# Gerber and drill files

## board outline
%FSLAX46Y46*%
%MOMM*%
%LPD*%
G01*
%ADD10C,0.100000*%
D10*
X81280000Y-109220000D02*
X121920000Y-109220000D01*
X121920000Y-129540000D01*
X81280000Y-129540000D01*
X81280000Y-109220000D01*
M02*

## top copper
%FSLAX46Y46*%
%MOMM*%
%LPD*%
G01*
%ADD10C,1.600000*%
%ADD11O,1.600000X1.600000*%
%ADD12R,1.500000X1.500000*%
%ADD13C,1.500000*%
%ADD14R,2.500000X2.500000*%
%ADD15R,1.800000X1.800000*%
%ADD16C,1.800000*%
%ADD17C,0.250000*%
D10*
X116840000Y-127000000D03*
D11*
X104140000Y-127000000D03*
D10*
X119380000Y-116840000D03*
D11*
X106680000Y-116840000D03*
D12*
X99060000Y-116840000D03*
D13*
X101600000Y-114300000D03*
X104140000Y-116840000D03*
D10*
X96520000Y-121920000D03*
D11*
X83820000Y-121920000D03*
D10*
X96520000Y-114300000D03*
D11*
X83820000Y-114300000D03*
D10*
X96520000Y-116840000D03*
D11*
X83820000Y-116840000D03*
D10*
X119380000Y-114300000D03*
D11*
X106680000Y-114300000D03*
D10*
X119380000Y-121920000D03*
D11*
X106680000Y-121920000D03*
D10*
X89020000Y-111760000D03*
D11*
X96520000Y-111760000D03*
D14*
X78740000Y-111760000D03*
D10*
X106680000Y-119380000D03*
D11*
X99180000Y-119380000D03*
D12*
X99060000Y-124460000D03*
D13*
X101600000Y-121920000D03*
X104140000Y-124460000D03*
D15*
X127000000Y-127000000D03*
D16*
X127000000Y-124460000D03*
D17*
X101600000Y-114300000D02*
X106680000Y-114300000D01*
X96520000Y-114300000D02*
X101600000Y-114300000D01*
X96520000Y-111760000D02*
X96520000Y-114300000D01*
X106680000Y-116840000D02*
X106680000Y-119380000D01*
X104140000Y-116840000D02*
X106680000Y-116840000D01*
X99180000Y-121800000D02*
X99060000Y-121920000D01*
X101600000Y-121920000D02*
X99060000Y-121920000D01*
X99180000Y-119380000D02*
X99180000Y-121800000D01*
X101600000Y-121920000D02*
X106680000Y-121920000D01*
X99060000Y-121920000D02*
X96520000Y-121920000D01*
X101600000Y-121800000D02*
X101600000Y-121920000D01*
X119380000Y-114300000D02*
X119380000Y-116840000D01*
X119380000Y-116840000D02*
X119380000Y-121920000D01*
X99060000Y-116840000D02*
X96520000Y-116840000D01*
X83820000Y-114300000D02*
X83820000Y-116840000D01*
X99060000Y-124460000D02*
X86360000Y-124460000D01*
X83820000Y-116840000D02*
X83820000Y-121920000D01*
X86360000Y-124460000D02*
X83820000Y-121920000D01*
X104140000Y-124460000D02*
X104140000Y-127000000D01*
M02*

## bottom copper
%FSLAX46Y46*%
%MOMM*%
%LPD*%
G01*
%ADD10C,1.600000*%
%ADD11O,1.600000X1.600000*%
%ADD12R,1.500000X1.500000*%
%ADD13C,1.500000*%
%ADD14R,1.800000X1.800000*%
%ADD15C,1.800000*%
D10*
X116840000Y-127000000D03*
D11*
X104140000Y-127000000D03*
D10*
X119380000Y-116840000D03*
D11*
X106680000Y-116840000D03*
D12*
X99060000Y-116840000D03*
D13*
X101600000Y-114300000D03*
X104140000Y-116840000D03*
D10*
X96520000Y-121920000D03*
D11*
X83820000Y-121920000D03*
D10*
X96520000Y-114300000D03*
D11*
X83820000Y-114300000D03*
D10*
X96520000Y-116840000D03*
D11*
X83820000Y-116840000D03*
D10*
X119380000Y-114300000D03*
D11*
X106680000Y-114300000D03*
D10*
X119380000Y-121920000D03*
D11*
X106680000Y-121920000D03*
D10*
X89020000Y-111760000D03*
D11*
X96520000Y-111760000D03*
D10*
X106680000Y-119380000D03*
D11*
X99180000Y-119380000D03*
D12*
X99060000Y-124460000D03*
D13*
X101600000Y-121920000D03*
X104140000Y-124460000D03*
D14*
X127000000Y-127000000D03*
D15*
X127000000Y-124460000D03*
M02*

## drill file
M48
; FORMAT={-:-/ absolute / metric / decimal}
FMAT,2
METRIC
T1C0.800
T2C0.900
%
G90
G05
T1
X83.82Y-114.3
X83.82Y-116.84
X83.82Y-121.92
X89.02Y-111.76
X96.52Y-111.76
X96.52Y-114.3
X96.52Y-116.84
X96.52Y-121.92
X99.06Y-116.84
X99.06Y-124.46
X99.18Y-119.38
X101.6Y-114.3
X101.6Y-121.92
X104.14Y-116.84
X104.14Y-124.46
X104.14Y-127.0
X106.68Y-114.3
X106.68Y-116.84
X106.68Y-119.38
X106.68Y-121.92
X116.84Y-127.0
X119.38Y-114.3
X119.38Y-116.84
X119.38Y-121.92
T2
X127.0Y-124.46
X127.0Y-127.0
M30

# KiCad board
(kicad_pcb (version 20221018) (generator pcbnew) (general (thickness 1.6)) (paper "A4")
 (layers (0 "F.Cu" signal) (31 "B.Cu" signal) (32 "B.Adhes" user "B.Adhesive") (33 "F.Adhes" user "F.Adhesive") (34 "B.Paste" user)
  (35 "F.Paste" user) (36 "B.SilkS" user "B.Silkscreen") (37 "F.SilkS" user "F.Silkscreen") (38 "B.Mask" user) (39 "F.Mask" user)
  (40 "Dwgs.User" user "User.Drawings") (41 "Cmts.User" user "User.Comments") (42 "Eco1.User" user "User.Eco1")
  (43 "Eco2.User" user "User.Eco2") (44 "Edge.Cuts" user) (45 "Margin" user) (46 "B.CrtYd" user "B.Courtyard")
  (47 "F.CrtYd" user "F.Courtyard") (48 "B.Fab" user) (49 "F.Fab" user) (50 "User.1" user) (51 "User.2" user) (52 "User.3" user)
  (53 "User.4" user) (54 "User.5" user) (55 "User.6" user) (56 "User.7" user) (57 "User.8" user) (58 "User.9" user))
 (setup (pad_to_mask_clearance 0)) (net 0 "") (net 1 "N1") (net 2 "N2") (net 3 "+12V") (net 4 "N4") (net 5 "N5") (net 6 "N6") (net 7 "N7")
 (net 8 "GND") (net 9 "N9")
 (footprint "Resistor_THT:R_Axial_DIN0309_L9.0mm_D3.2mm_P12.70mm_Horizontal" (layer "F.Cu") (at 116.84 127 180)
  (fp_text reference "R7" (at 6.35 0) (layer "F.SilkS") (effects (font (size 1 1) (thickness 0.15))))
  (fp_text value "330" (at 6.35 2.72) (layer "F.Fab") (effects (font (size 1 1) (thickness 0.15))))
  (pad "1" thru_hole circle (at 0 0 180) (size 1.6 1.6) (drill 0.8) (layers "*.Cu" "*.Mask") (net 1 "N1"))
  (pad "2" thru_hole oval (at 12.7 0 180) (size 1.6 1.6) (drill 0.8) (layers "*.Cu" "*.Mask") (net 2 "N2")))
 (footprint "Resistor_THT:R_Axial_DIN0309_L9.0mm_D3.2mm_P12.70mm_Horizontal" (layer "F.Cu") (at 119.38 116.84 180)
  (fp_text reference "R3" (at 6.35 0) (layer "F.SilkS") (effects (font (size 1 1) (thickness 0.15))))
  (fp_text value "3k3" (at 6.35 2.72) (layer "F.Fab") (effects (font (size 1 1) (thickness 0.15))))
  (pad "1" thru_hole circle (at 0 0 180) (size 1.6 1.6) (drill 0.8) (layers "*.Cu" "*.Mask") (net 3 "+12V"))
  (pad "2" thru_hole oval (at 12.7 0 180) (size 1.6 1.6) (drill 0.8) (layers "*.Cu" "*.Mask") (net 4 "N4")))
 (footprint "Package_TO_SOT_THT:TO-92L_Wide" (layer "F.Cu") (at 99.06 116.84)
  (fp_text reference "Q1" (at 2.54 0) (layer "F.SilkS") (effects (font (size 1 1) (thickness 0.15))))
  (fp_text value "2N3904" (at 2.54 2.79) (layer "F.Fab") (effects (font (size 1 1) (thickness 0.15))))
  (pad "1" thru_hole rect (at 0 0) (size 1.5 1.5) (drill 0.8) (layers "*.Cu" "*.Mask") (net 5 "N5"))
  (pad "2" thru_hole circle (at 2.54 -2.54) (size 1.5 1.5) (drill 0.8) (layers "*.Cu" "*.Mask") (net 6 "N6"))
  (pad "3" thru_hole circle (at 5.08 0) (size 1.5 1.5) (drill 0.8) (layers "*.Cu" "*.Mask") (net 4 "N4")))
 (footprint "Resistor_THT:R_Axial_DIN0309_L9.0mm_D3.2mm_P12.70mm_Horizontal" (layer "F.Cu") (at 96.52 121.92 180)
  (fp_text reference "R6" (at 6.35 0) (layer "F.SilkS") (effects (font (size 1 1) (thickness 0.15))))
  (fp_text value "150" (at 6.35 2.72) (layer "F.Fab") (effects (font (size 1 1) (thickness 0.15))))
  (pad "1" thru_hole circle (at 0 0 180) (size 1.6 1.6) (drill 0.8) (layers "*.Cu" "*.Mask") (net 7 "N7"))
  (pad "2" thru_hole oval (at 12.7 0 180) (size 1.6 1.6) (drill 0.8) (layers "*.Cu" "*.Mask") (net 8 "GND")))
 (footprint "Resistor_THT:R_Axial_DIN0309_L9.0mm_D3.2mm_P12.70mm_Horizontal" (layer "F.Cu") (at 96.52 114.3 180)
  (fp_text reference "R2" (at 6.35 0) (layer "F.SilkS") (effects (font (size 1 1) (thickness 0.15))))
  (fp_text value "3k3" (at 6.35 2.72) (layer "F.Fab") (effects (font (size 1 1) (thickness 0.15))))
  (pad "1" thru_hole circle (at 0 0 180) (size 1.6 1.6) (drill 0.8) (layers "*.Cu" "*.Mask") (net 6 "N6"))
  (pad "2" thru_hole oval (at 12.7 0 180) (size 1.6 1.6) (drill 0.8) (layers "*.Cu" "*.Mask") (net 8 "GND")))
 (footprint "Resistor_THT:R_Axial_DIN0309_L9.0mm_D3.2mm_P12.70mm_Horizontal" (layer "F.Cu") (at 96.52 116.84 180)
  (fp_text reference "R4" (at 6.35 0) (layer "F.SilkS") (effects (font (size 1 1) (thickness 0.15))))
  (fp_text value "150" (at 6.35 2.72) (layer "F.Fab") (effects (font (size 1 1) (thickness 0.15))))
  (pad "1" thru_hole circle (at 0 0 180) (size 1.6 1.6) (drill 0.8) (layers "*.Cu" "*.Mask") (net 5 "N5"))
  (pad "2" thru_hole oval (at 12.7 0 180) (size 1.6 1.6) (drill 0.8) (layers "*.Cu" "*.Mask") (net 8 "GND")))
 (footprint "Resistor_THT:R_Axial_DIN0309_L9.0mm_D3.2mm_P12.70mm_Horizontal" (layer "F.Cu") (at 119.38 114.3 180)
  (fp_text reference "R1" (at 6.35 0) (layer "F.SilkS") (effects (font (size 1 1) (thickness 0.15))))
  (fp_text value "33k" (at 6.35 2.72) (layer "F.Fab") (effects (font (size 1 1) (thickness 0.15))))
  (pad "1" thru_hole circle (at 0 0 180) (size 1.6 1.6) (drill 0.8) (layers "*.Cu" "*.Mask") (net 3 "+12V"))
  (pad "2" thru_hole oval (at 12.7 0 180) (size 1.6 1.6) (drill 0.8) (layers "*.Cu" "*.Mask") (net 6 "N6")))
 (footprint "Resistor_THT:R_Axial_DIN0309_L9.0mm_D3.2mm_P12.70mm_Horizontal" (layer "F.Cu") (at 119.38 121.92 180)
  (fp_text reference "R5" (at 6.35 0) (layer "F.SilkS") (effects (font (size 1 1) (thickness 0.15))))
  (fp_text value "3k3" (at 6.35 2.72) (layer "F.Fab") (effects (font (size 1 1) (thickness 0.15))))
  (pad "1" thru_hole circle (at 0 0 180) (size 1.6 1.6) (drill 0.8) (layers "*.Cu" "*.Mask") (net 3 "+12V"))
  (pad "2" thru_hole oval (at 12.7 0 180) (size 1.6 1.6) (drill 0.8) (layers "*.Cu" "*.Mask") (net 7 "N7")))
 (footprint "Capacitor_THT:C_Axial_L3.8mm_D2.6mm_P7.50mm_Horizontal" (layer "F.Cu") (at 89.02 111.76)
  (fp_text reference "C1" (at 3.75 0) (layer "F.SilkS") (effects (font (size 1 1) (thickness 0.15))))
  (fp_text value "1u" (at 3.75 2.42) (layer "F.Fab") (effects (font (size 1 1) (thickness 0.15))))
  (pad "1" thru_hole circle (at 0 0) (size 1.6 1.6) (drill 0.8) (layers "*.Cu" "*.Mask") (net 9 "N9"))
  (pad "2" thru_hole oval (at 7.5 0) (size 1.6 1.6) (drill 0.8) (layers "*.Cu" "*.Mask") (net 6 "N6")))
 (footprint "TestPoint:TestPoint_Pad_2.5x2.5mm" (layer "F.Cu") (at 78.74 111.76)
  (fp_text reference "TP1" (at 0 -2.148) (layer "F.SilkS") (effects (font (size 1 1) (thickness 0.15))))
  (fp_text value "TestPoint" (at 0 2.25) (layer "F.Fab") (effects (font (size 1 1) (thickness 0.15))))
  (pad "1" smd rect (at 0 0) (size 2.5 2.5) (layers "F.Cu" "F.Mask") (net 9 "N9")))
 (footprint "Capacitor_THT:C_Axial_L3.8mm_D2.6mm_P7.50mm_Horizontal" (layer "F.Cu") (at 106.68 119.38 180)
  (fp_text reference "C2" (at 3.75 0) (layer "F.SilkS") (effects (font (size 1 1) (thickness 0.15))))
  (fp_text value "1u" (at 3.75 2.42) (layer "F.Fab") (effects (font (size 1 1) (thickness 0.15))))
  (pad "1" thru_hole circle (at 0 0 180) (size 1.6 1.6) (drill 0.8) (layers "*.Cu" "*.Mask") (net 4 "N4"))
  (pad "2" thru_hole oval (at 7.5 0 180) (size 1.6 1.6) (drill 0.8) (layers "*.Cu" "*.Mask") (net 7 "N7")))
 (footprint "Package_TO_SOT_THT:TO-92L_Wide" (layer "F.Cu") (at 99.06 124.46)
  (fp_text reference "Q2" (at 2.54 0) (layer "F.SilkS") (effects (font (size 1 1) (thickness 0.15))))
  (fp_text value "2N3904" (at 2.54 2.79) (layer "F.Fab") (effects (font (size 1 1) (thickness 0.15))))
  (pad "1" thru_hole rect (at 0 0) (size 1.5 1.5) (drill 0.8) (layers "*.Cu" "*.Mask") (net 8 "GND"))
  (pad "2" thru_hole circle (at 2.54 -2.54) (size 1.5 1.5) (drill 0.8) (layers "*.Cu" "*.Mask") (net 7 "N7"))
  (pad "3" thru_hole circle (at 5.08 0) (size 1.5 1.5) (drill 0.8) (layers "*.Cu" "*.Mask") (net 2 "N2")))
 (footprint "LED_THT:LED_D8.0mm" (layer "F.Cu") (at 127 127 90)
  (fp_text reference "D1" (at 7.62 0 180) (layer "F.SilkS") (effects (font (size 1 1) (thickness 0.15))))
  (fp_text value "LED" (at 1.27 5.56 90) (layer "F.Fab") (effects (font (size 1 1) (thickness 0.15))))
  (pad "1" thru_hole rect (at 0 0 90) (size 1.8 1.8) (drill 0.9) (layers "*.Cu" "*.Mask") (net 1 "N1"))
  (pad "2" thru_hole circle (at 2.54 0 90) (size 1.8 1.8) (drill 0.9) (layers "*.Cu" "*.Mask") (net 3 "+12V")))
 (gr_rect (start 121.92 109.22) (end 81.28 129.54) (stroke (width 0.1) (type default)) (fill none) (layer "Edge.Cuts"))
 (segment (start 101.6 114.3) (end 106.68 114.3) (width 0.25) (layer "F.Cu") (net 6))
 (segment (start 96.52 114.3) (end 101.6 114.3) (width 0.25) (layer "F.Cu") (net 6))
 (segment (start 96.52 111.76) (end 96.52 114.3) (width 0.25) (layer "F.Cu") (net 6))
 (segment (start 106.68 116.84) (end 106.68 119.38) (width 0.25) (layer "F.Cu") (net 4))
 (segment (start 104.14 116.84) (end 106.68 116.84) (width 0.25) (layer "F.Cu") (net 4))
 (segment (start 99.18 121.8) (end 99.06 121.92) (width 0.25) (layer "F.Cu") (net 7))
 (segment (start 101.6 121.92) (end 99.06 121.92) (width 0.25) (layer "F.Cu") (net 7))
 (segment (start 99.18 119.38) (end 99.18 121.8) (width 0.25) (layer "F.Cu") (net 7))
 (segment (start 101.6 121.92) (end 106.68 121.92) (width 0.25) (layer "F.Cu") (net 7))
 (segment (start 99.06 121.92) (end 96.52 121.92) (width 0.25) (layer "F.Cu") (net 7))
 (segment (start 101.6 121.8) (end 101.6 121.92) (width 0.25) (layer "F.Cu") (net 7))
 (segment (start 119.38 114.3) (end 119.38 116.84) (width 0.25) (layer "F.Cu") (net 3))
 (segment (start 119.38 116.84) (end 119.38 121.92) (width 0.25) (layer "F.Cu") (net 3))
 (segment (start 99.06 116.84) (end 96.52 116.84) (width 0.25) (layer "F.Cu") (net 5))
 (segment (start 83.82 114.3) (end 83.82 116.84) (width 0.25) (layer "F.Cu") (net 8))
 (segment (start 99.06 124.46) (end 86.36 124.46) (width 0.25) (layer "F.Cu") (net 8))
 (segment (start 83.82 116.84) (end 83.82 121.92) (width 0.25) (layer "F.Cu") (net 8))
 (segment (start 86.36 124.46) (end 83.82 121.92) (width 0.25) (layer "F.Cu") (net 8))
 (segment (start 104.14 124.46) (end 104.14 127) (width 0.25) (layer "F.Cu") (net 2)))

